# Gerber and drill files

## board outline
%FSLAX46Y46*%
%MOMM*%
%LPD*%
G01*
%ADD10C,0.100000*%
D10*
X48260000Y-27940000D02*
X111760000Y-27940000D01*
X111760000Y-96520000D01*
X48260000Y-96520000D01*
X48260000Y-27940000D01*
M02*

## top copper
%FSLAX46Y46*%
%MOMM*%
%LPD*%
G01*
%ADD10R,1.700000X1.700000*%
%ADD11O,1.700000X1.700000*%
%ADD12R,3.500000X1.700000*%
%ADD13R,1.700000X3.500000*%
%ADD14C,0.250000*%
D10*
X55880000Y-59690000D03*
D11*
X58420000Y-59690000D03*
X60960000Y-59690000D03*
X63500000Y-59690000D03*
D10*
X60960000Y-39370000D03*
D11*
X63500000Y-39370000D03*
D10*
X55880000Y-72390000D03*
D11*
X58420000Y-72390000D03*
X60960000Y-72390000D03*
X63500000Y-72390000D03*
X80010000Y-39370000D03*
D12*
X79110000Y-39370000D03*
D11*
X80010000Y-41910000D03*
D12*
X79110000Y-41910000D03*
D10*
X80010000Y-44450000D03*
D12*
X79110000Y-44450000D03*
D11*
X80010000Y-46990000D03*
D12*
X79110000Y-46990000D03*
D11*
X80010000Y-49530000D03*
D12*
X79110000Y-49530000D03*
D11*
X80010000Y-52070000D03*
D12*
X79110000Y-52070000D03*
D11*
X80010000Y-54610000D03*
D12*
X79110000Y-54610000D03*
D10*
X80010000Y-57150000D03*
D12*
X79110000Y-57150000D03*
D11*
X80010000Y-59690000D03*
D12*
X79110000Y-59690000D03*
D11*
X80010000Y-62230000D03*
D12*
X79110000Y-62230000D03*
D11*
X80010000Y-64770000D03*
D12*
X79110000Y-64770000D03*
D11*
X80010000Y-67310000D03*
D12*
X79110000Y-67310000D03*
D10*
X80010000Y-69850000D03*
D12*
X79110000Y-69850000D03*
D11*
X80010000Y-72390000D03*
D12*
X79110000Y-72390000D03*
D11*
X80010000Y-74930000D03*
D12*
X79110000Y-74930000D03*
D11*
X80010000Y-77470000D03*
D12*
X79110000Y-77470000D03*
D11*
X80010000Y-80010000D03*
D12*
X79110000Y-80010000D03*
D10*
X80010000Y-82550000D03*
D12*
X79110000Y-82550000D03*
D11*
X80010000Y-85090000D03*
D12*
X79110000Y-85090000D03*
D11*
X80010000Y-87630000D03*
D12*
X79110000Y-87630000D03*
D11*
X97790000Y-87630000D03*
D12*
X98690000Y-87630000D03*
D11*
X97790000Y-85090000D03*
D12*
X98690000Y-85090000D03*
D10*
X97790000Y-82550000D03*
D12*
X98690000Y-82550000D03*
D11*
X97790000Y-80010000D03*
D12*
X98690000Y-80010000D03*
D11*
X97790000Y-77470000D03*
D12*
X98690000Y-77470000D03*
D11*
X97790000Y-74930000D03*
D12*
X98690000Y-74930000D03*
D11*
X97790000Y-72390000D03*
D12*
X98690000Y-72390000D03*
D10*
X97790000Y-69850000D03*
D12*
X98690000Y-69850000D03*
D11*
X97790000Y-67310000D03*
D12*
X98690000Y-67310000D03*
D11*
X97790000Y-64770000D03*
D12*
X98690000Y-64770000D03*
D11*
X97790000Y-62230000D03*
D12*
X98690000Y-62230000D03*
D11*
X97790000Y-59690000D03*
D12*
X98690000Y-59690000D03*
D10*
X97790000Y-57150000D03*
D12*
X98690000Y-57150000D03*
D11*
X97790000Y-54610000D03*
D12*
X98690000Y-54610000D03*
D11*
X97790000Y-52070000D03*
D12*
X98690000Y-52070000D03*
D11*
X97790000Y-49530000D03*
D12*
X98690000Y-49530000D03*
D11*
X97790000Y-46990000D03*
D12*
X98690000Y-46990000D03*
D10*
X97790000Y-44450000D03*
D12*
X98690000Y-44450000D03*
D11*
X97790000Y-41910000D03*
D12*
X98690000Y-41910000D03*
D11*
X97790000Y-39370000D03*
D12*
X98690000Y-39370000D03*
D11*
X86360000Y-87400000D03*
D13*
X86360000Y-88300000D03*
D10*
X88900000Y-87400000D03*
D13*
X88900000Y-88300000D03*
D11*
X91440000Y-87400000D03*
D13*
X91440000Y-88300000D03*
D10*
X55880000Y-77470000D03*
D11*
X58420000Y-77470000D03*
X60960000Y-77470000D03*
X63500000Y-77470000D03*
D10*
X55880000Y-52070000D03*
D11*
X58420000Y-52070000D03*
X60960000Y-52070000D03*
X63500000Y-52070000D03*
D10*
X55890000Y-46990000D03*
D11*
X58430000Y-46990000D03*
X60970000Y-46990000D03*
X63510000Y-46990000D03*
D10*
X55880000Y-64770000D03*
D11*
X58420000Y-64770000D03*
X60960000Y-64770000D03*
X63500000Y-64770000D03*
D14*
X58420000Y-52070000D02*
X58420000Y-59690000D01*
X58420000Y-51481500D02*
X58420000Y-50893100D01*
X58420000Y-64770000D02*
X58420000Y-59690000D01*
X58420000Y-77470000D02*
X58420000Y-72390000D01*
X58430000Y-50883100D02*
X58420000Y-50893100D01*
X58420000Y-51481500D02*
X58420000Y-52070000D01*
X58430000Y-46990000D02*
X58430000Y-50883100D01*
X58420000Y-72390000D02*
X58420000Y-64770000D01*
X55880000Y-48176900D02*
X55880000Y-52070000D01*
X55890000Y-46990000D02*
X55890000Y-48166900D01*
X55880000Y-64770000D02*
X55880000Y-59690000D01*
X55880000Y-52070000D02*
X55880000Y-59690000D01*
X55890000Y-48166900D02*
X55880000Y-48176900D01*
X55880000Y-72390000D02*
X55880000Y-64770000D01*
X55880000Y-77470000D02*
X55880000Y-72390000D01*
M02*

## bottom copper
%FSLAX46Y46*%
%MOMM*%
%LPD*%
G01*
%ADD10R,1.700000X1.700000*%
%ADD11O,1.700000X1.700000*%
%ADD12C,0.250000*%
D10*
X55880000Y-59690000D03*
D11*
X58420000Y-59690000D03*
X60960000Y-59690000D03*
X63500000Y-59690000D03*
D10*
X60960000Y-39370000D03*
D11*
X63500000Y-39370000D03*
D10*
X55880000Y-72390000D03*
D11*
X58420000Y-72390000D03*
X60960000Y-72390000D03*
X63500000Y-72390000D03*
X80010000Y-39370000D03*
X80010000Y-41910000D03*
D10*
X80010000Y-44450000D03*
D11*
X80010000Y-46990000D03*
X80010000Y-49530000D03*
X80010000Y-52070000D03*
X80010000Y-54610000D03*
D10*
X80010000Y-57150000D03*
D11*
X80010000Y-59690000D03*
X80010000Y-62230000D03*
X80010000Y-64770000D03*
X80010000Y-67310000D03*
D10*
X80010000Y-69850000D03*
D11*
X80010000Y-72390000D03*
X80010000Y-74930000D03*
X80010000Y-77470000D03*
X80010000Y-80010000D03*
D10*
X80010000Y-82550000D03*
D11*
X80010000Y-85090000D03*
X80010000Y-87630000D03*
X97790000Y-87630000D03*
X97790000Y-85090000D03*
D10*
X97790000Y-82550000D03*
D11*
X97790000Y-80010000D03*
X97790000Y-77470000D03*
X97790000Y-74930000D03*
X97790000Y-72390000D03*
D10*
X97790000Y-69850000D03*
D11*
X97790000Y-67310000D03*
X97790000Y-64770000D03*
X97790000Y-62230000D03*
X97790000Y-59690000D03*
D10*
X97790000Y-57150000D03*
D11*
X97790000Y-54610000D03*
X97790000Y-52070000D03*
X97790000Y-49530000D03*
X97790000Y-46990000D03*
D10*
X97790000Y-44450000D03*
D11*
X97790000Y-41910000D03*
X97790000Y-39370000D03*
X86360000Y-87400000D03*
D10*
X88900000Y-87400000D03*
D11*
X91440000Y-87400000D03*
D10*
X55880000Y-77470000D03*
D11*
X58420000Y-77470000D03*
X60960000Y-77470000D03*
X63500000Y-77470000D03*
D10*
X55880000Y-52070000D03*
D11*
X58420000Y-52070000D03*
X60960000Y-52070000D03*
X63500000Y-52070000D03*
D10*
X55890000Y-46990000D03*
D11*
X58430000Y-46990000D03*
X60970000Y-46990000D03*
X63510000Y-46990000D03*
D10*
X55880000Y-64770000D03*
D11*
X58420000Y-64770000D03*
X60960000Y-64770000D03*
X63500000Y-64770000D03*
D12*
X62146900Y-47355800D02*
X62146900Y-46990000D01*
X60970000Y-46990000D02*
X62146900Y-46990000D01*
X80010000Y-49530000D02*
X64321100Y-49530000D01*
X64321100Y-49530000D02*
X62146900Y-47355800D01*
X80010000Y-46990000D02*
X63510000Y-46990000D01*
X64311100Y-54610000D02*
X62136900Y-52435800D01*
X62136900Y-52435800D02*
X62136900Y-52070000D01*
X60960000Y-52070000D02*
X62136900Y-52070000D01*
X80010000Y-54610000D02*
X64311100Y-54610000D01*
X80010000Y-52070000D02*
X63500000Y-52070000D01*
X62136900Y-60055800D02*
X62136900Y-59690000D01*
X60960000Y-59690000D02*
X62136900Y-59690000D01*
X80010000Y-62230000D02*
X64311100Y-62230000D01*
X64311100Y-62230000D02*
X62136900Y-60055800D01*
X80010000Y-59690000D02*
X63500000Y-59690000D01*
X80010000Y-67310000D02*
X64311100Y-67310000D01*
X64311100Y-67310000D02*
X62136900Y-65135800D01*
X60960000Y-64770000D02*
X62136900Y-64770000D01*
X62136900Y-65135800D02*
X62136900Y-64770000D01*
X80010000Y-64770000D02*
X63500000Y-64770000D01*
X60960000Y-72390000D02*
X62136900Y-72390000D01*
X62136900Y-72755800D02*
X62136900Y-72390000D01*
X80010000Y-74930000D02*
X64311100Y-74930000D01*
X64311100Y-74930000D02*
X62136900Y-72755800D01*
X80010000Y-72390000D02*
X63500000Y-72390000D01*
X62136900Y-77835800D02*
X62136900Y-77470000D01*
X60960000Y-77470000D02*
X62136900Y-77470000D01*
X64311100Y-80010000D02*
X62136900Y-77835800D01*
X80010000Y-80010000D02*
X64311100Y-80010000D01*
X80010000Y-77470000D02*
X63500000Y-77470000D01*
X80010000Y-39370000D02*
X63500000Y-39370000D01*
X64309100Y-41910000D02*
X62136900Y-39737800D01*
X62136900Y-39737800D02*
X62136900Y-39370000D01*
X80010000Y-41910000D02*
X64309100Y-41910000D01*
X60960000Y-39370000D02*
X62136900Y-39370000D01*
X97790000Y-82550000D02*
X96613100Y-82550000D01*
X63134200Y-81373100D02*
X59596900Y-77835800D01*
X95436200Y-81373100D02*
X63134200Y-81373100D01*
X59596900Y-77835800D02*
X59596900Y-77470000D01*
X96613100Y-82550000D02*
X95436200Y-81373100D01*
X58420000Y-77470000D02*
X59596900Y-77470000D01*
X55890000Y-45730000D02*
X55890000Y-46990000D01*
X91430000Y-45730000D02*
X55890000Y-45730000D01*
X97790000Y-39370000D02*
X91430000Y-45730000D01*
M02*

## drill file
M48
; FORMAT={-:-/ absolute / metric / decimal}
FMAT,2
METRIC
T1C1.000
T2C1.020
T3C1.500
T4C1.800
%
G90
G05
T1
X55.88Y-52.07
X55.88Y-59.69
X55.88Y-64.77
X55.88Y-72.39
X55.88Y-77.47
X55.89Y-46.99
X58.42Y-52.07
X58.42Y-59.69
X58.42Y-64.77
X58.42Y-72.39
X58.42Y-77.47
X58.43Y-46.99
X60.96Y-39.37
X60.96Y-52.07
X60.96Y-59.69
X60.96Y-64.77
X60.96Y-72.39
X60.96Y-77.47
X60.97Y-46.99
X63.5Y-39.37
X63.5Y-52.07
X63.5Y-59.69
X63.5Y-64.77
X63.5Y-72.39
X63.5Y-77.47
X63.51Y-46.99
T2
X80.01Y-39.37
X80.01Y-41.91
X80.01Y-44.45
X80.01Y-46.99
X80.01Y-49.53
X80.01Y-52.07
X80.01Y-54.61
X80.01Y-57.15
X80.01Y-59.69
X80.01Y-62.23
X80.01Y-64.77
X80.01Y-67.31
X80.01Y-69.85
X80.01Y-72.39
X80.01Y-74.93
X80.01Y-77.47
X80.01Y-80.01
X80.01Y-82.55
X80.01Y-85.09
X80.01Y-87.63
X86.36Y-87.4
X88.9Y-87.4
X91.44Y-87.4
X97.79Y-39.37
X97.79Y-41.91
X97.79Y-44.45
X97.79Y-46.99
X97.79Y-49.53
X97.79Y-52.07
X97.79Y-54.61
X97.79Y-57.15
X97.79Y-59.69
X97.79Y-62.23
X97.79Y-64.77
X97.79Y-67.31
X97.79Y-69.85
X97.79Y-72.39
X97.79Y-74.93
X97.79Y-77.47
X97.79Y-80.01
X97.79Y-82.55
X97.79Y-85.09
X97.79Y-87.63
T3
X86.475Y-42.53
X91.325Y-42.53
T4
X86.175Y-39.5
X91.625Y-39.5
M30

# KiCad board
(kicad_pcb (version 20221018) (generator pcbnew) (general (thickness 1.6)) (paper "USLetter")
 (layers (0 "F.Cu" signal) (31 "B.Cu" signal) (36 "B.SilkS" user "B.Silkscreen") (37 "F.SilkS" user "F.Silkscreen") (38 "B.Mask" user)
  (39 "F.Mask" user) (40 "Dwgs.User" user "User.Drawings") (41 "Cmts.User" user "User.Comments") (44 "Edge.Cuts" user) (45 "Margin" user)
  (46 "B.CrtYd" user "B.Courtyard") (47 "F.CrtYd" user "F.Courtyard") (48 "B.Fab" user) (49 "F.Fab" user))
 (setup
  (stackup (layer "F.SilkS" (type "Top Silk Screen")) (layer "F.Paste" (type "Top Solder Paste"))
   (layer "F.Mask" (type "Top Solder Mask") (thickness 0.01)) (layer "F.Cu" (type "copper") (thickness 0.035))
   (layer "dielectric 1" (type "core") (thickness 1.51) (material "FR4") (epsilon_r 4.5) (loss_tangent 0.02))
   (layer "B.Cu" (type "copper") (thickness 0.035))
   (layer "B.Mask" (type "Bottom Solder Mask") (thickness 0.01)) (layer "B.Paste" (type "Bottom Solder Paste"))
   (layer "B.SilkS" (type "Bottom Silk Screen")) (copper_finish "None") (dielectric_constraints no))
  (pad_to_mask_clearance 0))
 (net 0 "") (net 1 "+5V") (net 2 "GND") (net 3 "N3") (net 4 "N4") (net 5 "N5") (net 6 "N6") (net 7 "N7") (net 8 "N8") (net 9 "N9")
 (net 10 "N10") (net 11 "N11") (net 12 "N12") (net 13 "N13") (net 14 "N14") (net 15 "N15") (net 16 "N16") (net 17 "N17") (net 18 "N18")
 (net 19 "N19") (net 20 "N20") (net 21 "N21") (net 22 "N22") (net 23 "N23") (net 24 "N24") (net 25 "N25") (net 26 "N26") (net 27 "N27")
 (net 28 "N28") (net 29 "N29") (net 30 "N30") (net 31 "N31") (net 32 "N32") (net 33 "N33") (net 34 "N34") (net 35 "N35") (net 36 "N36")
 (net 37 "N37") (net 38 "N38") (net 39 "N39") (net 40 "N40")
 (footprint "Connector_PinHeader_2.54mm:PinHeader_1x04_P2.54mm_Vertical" (layer "F.Cu") (at 55.88 59.69 90)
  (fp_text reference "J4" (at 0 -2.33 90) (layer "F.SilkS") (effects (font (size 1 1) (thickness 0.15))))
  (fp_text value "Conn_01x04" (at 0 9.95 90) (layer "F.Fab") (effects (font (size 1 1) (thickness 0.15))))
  (pad "1" thru_hole rect (at 0 0 90) (size 1.7 1.7) (drill 1) (layers "*.Cu" "*.Mask") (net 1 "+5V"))
  (pad "2" thru_hole oval (at 0 2.54 90) (size 1.7 1.7) (drill 1) (layers "*.Cu" "*.Mask") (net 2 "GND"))
  (pad "3" thru_hole oval (at 0 5.08 90) (size 1.7 1.7) (drill 1) (layers "*.Cu" "*.Mask") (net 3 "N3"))
  (pad "4" thru_hole oval (at 0 7.62 90) (size 1.7 1.7) (drill 1) (layers "*.Cu" "*.Mask") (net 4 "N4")))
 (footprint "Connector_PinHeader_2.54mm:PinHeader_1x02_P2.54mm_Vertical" (layer "F.Cu") (at 60.96 39.37 90)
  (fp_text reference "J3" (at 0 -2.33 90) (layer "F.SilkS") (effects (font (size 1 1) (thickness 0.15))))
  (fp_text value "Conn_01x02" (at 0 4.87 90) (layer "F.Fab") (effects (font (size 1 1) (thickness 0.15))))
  (pad "1" thru_hole rect (at 0 0 90) (size 1.7 1.7) (drill 1) (layers "*.Cu" "*.Mask") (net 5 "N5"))
  (pad "2" thru_hole oval (at 0 2.54 90) (size 1.7 1.7) (drill 1) (layers "*.Cu" "*.Mask") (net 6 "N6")))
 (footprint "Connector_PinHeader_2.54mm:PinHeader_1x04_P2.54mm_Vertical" (layer "F.Cu") (at 55.88 72.39 90)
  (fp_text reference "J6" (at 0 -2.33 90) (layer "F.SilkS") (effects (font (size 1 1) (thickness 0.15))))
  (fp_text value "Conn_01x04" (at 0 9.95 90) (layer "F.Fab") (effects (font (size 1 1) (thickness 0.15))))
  (pad "1" thru_hole rect (at 0 0 90) (size 1.7 1.7) (drill 1) (layers "*.Cu" "*.Mask") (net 1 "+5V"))
  (pad "2" thru_hole oval (at 0 2.54 90) (size 1.7 1.7) (drill 1) (layers "*.Cu" "*.Mask") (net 2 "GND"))
  (pad "3" thru_hole oval (at 0 5.08 90) (size 1.7 1.7) (drill 1) (layers "*.Cu" "*.Mask") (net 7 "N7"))
  (pad "4" thru_hole oval (at 0 7.62 90) (size 1.7 1.7) (drill 1) (layers "*.Cu" "*.Mask") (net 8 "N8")))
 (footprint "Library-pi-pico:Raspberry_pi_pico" (layer "F.Cu") (at 91.794 24.13)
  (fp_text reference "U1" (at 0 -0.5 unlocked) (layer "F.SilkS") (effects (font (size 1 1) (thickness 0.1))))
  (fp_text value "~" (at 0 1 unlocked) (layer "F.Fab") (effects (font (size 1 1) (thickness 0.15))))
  (pad "" np_thru_hole oval (at -5.619 15.37) (size 1.8 1.8) (drill 1.8) (layers "*.Cu" "*.Mask"))
  (pad "" np_thru_hole oval (at -5.319 18.4) (size 1.5 1.5) (drill 1.5) (layers "*.Cu" "*.Mask"))
  (pad "" np_thru_hole oval (at -0.469 18.4) (size 1.5 1.5) (drill 1.5) (layers "*.Cu" "*.Mask"))
  (pad "" np_thru_hole oval (at -0.169 15.37) (size 1.8 1.8) (drill 1.8) (layers "*.Cu" "*.Mask"))
  (pad "1" thru_hole oval (at -11.784 15.24) (size 1.7 1.7) (drill 1.02) (layers "*.Cu" "*.Mask") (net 6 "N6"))
  (pad "1" smd rect (at -11.784 15.24) (size 3.5 1.7) (drill (offset -0.9 0)) (layers "F.Cu" "F.Mask") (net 6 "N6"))
  (pad "2" thru_hole oval (at -11.784 17.78) (size 1.7 1.7) (drill 1.02) (layers "*.Cu" "*.Mask") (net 5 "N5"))
  (pad "2" smd rect (at -11.784 17.78) (size 3.5 1.7) (drill (offset -0.9 0)) (layers "F.Cu" "F.Mask") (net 5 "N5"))
  (pad "3" thru_hole rect (at -11.784 20.32) (size 1.7 1.7) (drill 1.02) (layers "*.Cu" "*.Mask") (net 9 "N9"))
  (pad "3" smd rect (at -11.784 20.32) (size 3.5 1.7) (drill (offset -0.9 0)) (layers "F.Cu" "F.Mask") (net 9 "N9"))
  (pad "4" thru_hole oval (at -11.784 22.86) (size 1.7 1.7) (drill 1.02) (layers "*.Cu" "*.Mask") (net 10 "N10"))
  (pad "4" smd rect (at -11.784 22.86) (size 3.5 1.7) (drill (offset -0.9 0)) (layers "F.Cu" "F.Mask") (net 10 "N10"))
  (pad "5" thru_hole oval (at -11.784 25.4) (size 1.7 1.7) (drill 1.02) (layers "*.Cu" "*.Mask") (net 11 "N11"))
  (pad "5" smd rect (at -11.784 25.4) (size 3.5 1.7) (drill (offset -0.9 0)) (layers "F.Cu" "F.Mask") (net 11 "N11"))
  (pad "6" thru_hole oval (at -11.784 27.94) (size 1.7 1.7) (drill 1.02) (layers "*.Cu" "*.Mask") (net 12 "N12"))
  (pad "6" smd rect (at -11.784 27.94) (size 3.5 1.7) (drill (offset -0.9 0)) (layers "F.Cu" "F.Mask") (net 12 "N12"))
  (pad "7" thru_hole oval (at -11.784 30.48) (size 1.7 1.7) (drill 1.02) (layers "*.Cu" "*.Mask") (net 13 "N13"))
  (pad "7" smd rect (at -11.784 30.48) (size 3.5 1.7) (drill (offset -0.9 0)) (layers "F.Cu" "F.Mask") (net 13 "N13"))
  (pad "8" thru_hole rect (at -11.784 33.02) (size 1.7 1.7) (drill 1.02) (layers "*.Cu" "*.Mask") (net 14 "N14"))
  (pad "8" smd rect (at -11.784 33.02) (size 3.5 1.7) (drill (offset -0.9 0)) (layers "F.Cu" "F.Mask") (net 14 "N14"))
  (pad "9" thru_hole oval (at -11.784 35.56) (size 1.7 1.7) (drill 1.02) (layers "*.Cu" "*.Mask") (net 4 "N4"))
  (pad "9" smd rect (at -11.784 35.56) (size 3.5 1.7) (drill (offset -0.9 0)) (layers "F.Cu" "F.Mask") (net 4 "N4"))
  (pad "10" thru_hole oval (at -11.784 38.1) (size 1.7 1.7) (drill 1.02) (layers "*.Cu" "*.Mask") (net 3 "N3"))
  (pad "10" smd rect (at -11.784 38.1) (size 3.5 1.7) (drill (offset -0.9 0)) (layers "F.Cu" "F.Mask") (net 3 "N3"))
  (pad "11" thru_hole oval (at -11.784 40.64) (size 1.7 1.7) (drill 1.02) (layers "*.Cu" "*.Mask") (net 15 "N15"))
  (pad "11" smd rect (at -11.784 40.64) (size 3.5 1.7) (drill (offset -0.9 0)) (layers "F.Cu" "F.Mask") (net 15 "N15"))
  (pad "12" thru_hole oval (at -11.784 43.18) (size 1.7 1.7) (drill 1.02) (layers "*.Cu" "*.Mask") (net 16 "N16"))
  (pad "12" smd rect (at -11.784 43.18) (size 3.5 1.7) (drill (offset -0.9 0)) (layers "F.Cu" "F.Mask") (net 16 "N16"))
  (pad "13" thru_hole rect (at -11.784 45.72) (size 1.7 1.7) (drill 1.02) (layers "*.Cu" "*.Mask") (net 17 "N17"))
  (pad "13" smd rect (at -11.784 45.72) (size 3.5 1.7) (drill (offset -0.9 0)) (layers "F.Cu" "F.Mask") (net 17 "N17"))
  (pad "14" thru_hole oval (at -11.784 48.26) (size 1.7 1.7) (drill 1.02) (layers "*.Cu" "*.Mask") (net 8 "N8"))
  (pad "14" smd rect (at -11.784 48.26) (size 3.5 1.7) (drill (offset -0.9 0)) (layers "F.Cu" "F.Mask") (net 8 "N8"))
  (pad "15" thru_hole oval (at -11.784 50.8) (size 1.7 1.7) (drill 1.02) (layers "*.Cu" "*.Mask") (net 7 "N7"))
  (pad "15" smd rect (at -11.784 50.8) (size 3.5 1.7) (drill (offset -0.9 0)) (layers "F.Cu" "F.Mask") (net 7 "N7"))
  (pad "16" thru_hole oval (at -11.784 53.34) (size 1.7 1.7) (drill 1.02) (layers "*.Cu" "*.Mask") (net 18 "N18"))
  (pad "16" smd rect (at -11.784 53.34) (size 3.5 1.7) (drill (offset -0.9 0)) (layers "F.Cu" "F.Mask") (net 18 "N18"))
  (pad "17" thru_hole oval (at -11.784 55.88) (size 1.7 1.7) (drill 1.02) (layers "*.Cu" "*.Mask") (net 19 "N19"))
  (pad "17" smd rect (at -11.784 55.88) (size 3.5 1.7) (drill (offset -0.9 0)) (layers "F.Cu" "F.Mask") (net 19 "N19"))
  (pad "18" thru_hole rect (at -11.784 58.42) (size 1.7 1.7) (drill 1.02) (layers "*.Cu" "*.Mask") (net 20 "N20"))
  (pad "18" smd rect (at -11.784 58.42) (size 3.5 1.7) (drill (offset -0.9 0)) (layers "F.Cu" "F.Mask") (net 20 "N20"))
  (pad "19" thru_hole oval (at -11.784 60.96) (size 1.7 1.7) (drill 1.02) (layers "*.Cu" "*.Mask") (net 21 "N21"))
  (pad "19" smd rect (at -11.784 60.96) (size 3.5 1.7) (drill (offset -0.9 0)) (layers "F.Cu" "F.Mask") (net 21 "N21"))
  (pad "20" thru_hole oval (at -11.784 63.5) (size 1.7 1.7) (drill 1.02) (layers "*.Cu" "*.Mask") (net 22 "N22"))
  (pad "20" smd rect (at -11.784 63.5) (size 3.5 1.7) (drill (offset -0.9 0)) (layers "F.Cu" "F.Mask") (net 22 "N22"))
  (pad "21" thru_hole oval (at 5.996 63.5) (size 1.7 1.7) (drill 1.02) (layers "*.Cu" "*.Mask") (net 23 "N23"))
  (pad "21" smd rect (at 5.996 63.5) (size 3.5 1.7) (drill (offset 0.9 0)) (layers "F.Cu" "F.Mask") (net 23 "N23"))
  (pad "22" thru_hole oval (at 5.996 60.96) (size 1.7 1.7) (drill 1.02) (layers "*.Cu" "*.Mask") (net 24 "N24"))
  (pad "22" smd rect (at 5.996 60.96) (size 3.5 1.7) (drill (offset 0.9 0)) (layers "F.Cu" "F.Mask") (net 24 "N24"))
  (pad "23" thru_hole rect (at 5.996 58.42) (size 1.7 1.7) (drill 1.02) (layers "*.Cu" "*.Mask") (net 2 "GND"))
  (pad "23" smd rect (at 5.996 58.42) (size 3.5 1.7) (drill (offset 0.9 0)) (layers "F.Cu" "F.Mask") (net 2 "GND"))
  (pad "24" thru_hole oval (at 5.996 55.88) (size 1.7 1.7) (drill 1.02) (layers "*.Cu" "*.Mask") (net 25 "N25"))
  (pad "24" smd rect (at 5.996 55.88) (size 3.5 1.7) (drill (offset 0.9 0)) (layers "F.Cu" "F.Mask") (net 25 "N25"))
  (pad "25" thru_hole oval (at 5.996 53.34) (size 1.7 1.7) (drill 1.02) (layers "*.Cu" "*.Mask") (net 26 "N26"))
  (pad "25" smd rect (at 5.996 53.34) (size 3.5 1.7) (drill (offset 0.9 0)) (layers "F.Cu" "F.Mask") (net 26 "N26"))
  (pad "26" thru_hole oval (at 5.996 50.8) (size 1.7 1.7) (drill 1.02) (layers "*.Cu" "*.Mask") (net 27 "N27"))
  (pad "26" smd rect (at 5.996 50.8) (size 3.5 1.7) (drill (offset 0.9 0)) (layers "F.Cu" "F.Mask") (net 27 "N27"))
  (pad "27" thru_hole oval (at 5.996 48.26) (size 1.7 1.7) (drill 1.02) (layers "*.Cu" "*.Mask") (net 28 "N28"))
  (pad "27" smd rect (at 5.996 48.26) (size 3.5 1.7) (drill (offset 0.9 0)) (layers "F.Cu" "F.Mask") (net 28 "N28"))
  (pad "28" thru_hole rect (at 5.996 45.72) (size 1.7 1.7) (drill 1.02) (layers "*.Cu" "*.Mask") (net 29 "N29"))
  (pad "28" smd rect (at 5.996 45.72) (size 3.5 1.7) (drill (offset 0.9 0)) (layers "F.Cu" "F.Mask") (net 29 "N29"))
  (pad "29" thru_hole oval (at 5.996 43.18) (size 1.7 1.7) (drill 1.02) (layers "*.Cu" "*.Mask") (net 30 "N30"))
  (pad "29" smd rect (at 5.996 43.18) (size 3.5 1.7) (drill (offset 0.9 0)) (layers "F.Cu" "F.Mask") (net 30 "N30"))
  (pad "30" thru_hole oval (at 5.996 40.64) (size 1.7 1.7) (drill 1.02) (layers "*.Cu" "*.Mask") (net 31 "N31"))
  (pad "30" smd rect (at 5.996 40.64) (size 3.5 1.7) (drill (offset 0.9 0)) (layers "F.Cu" "F.Mask") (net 31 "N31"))
  (pad "31" thru_hole oval (at 5.996 38.1) (size 1.7 1.7) (drill 1.02) (layers "*.Cu" "*.Mask") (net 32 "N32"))
  (pad "31" smd rect (at 5.996 38.1) (size 3.5 1.7) (drill (offset 0.9 0)) (layers "F.Cu" "F.Mask") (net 32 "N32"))
  (pad "32" thru_hole oval (at 5.996 35.56) (size 1.7 1.7) (drill 1.02) (layers "*.Cu" "*.Mask") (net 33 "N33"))
  (pad "32" smd rect (at 5.996 35.56) (size 3.5 1.7) (drill (offset 0.9 0)) (layers "F.Cu" "F.Mask") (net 33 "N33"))
  (pad "33" thru_hole rect (at 5.996 33.02) (size 1.7 1.7) (drill 1.02) (layers "*.Cu" "*.Mask") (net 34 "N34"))
  (pad "33" smd rect (at 5.996 33.02) (size 3.5 1.7) (drill (offset 0.9 0)) (layers "F.Cu" "F.Mask") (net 34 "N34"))
  (pad "34" thru_hole oval (at 5.996 30.48) (size 1.7 1.7) (drill 1.02) (layers "*.Cu" "*.Mask") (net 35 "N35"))
  (pad "34" smd rect (at 5.996 30.48) (size 3.5 1.7) (drill (offset 0.9 0)) (layers "F.Cu" "F.Mask") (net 35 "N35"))
  (pad "35" thru_hole oval (at 5.996 27.94) (size 1.7 1.7) (drill 1.02) (layers "*.Cu" "*.Mask") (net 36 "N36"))
  (pad "35" smd rect (at 5.996 27.94) (size 3.5 1.7) (drill (offset 0.9 0)) (layers "F.Cu" "F.Mask") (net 36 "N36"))
  (pad "36" thru_hole oval (at 5.996 25.4) (size 1.7 1.7) (drill 1.02) (layers "*.Cu" "*.Mask") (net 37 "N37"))
  (pad "36" smd rect (at 5.996 25.4) (size 3.5 1.7) (drill (offset 0.9 0)) (layers "F.Cu" "F.Mask") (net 37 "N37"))
  (pad "37" thru_hole oval (at 5.996 22.86) (size 1.7 1.7) (drill 1.02) (layers "*.Cu" "*.Mask") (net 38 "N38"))
  (pad "37" smd rect (at 5.996 22.86) (size 3.5 1.7) (drill (offset 0.9 0)) (layers "F.Cu" "F.Mask") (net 38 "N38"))
  (pad "38" thru_hole rect (at 5.996 20.32) (size 1.7 1.7) (drill 1.02) (layers "*.Cu" "*.Mask") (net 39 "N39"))
  (pad "38" smd rect (at 5.996 20.32) (size 3.5 1.7) (drill (offset 0.9 0)) (layers "F.Cu" "F.Mask") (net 39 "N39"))
  (pad "39" thru_hole oval (at 5.996 17.78) (size 1.7 1.7) (drill 1.02) (layers "*.Cu" "*.Mask") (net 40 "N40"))
  (pad "39" smd rect (at 5.996 17.78) (size 3.5 1.7) (drill (offset 0.9 0)) (layers "F.Cu" "F.Mask") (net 40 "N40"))
  (pad "40" thru_hole oval (at 5.996 15.24) (size 1.7 1.7) (drill 1.02) (layers "*.Cu" "*.Mask") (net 1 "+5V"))
  (pad "40" smd rect (at 5.996 15.24) (size 3.5 1.7) (drill (offset 0.9 0)) (layers "F.Cu" "F.Mask") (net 1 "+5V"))
  (pad "41" thru_hole oval (at -5.434 63.27) (size 1.7 1.7) (drill 1.02) (layers "*.Cu" "*.Mask"))
  (pad "41" smd rect (at -5.434 63.27 90) (size 3.5 1.7) (drill (offset -0.9 0)) (layers "F.Cu" "F.Mask"))
  (pad "42" thru_hole rect (at -2.894 63.27) (size 1.7 1.7) (drill 1.02) (layers "*.Cu" "*.Mask"))
  (pad "42" smd rect (at -2.894 63.27 90) (size 3.5 1.7) (drill (offset -0.9 0)) (layers "F.Cu" "F.Mask"))
  (pad "43" thru_hole oval (at -0.354 63.27) (size 1.7 1.7) (drill 1.02) (layers "*.Cu" "*.Mask"))
  (pad "43" smd rect (at -0.354 63.27 90) (size 3.5 1.7) (drill (offset -0.9 0)) (layers "F.Cu" "F.Mask")))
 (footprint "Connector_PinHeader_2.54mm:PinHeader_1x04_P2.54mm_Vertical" (layer "F.Cu") (at 55.88 77.47 90)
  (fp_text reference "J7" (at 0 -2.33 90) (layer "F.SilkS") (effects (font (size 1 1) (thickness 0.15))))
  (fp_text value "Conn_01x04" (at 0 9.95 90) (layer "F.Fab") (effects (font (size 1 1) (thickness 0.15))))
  (pad "1" thru_hole rect (at 0 0 90) (size 1.7 1.7) (drill 1) (layers "*.Cu" "*.Mask") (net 1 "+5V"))
  (pad "2" thru_hole oval (at 0 2.54 90) (size 1.7 1.7) (drill 1) (layers "*.Cu" "*.Mask") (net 2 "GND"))
  (pad "3" thru_hole oval (at 0 5.08 90) (size 1.7 1.7) (drill 1) (layers "*.Cu" "*.Mask") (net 19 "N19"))
  (pad "4" thru_hole oval (at 0 7.62 90) (size 1.7 1.7) (drill 1) (layers "*.Cu" "*.Mask") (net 18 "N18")))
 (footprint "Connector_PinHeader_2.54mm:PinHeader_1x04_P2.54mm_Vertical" (layer "F.Cu") (at 55.88 52.07 90)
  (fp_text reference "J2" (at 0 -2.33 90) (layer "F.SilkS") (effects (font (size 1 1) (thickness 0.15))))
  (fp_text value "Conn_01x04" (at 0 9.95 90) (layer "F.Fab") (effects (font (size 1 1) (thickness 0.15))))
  (pad "1" thru_hole rect (at 0 0 90) (size 1.7 1.7) (drill 1) (layers "*.Cu" "*.Mask") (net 1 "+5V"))
  (pad "2" thru_hole oval (at 0 2.54 90) (size 1.7 1.7) (drill 1) (layers "*.Cu" "*.Mask") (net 2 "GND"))
  (pad "3" thru_hole oval (at 0 5.08 90) (size 1.7 1.7) (drill 1) (layers "*.Cu" "*.Mask") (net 13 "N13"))
  (pad "4" thru_hole oval (at 0 7.62 90) (size 1.7 1.7) (drill 1) (layers "*.Cu" "*.Mask") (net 12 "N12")))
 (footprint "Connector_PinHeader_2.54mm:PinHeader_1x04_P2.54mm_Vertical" (layer "F.Cu") (at 55.89 46.99 90)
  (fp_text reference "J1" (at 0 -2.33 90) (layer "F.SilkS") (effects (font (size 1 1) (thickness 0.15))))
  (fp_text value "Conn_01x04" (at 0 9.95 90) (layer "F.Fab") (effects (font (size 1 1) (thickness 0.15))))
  (pad "1" thru_hole rect (at 0 0 90) (size 1.7 1.7) (drill 1) (layers "*.Cu" "*.Mask") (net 1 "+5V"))
  (pad "2" thru_hole oval (at 0 2.54 90) (size 1.7 1.7) (drill 1) (layers "*.Cu" "*.Mask") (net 2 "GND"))
  (pad "3" thru_hole oval (at 0 5.08 90) (size 1.7 1.7) (drill 1) (layers "*.Cu" "*.Mask") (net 11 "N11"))
  (pad "4" thru_hole oval (at 0 7.62 90) (size 1.7 1.7) (drill 1) (layers "*.Cu" "*.Mask") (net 10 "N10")))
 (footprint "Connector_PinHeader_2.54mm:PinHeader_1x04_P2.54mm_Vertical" (layer "F.Cu") (at 55.88 64.77 90)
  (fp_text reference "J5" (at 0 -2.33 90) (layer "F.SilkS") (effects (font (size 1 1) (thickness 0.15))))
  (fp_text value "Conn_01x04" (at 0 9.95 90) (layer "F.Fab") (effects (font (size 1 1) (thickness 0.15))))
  (pad "1" thru_hole rect (at 0 0 90) (size 1.7 1.7) (drill 1) (layers "*.Cu" "*.Mask") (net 1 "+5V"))
  (pad "2" thru_hole oval (at 0 2.54 90) (size 1.7 1.7) (drill 1) (layers "*.Cu" "*.Mask") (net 2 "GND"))
  (pad "3" thru_hole oval (at 0 5.08 90) (size 1.7 1.7) (drill 1) (layers "*.Cu" "*.Mask") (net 16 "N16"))
  (pad "4" thru_hole oval (at 0 7.62 90) (size 1.7 1.7) (drill 1) (layers "*.Cu" "*.Mask") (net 15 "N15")))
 (gr_rect (start 48.26 27.94) (end 111.76 96.52) (stroke (width 0.1) (type default)) (fill none) (layer "Edge.Cuts"))
 (segment (start 62.1469 47.3558) (end 62.1469 46.99) (width 0.25) (layer "B.Cu") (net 11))
 (segment (start 60.97 46.99) (end 62.1469 46.99) (width 0.25) (layer "B.Cu") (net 11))
 (segment (start 80.01 49.53) (end 64.3211 49.53) (width 0.25) (layer "B.Cu") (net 11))
 (segment (start 64.3211 49.53) (end 62.1469 47.3558) (width 0.25) (layer "B.Cu") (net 11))
 (segment (start 80.01 46.99) (end 63.51 46.99) (width 0.25) (layer "B.Cu") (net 10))
 (segment (start 64.3111 54.61) (end 62.1369 52.4358) (width 0.25) (layer "B.Cu") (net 13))
 (segment (start 62.1369 52.4358) (end 62.1369 52.07) (width 0.25) (layer "B.Cu") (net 13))
 (segment (start 60.96 52.07) (end 62.1369 52.07) (width 0.25) (layer "B.Cu") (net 13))
 (segment (start 80.01 54.61) (end 64.3111 54.61) (width 0.25) (layer "B.Cu") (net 13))
 (segment (start 80.01 52.07) (end 63.5 52.07) (width 0.25) (layer "B.Cu") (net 12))
 (segment (start 62.1369 60.0558) (end 62.1369 59.69) (width 0.25) (layer "B.Cu") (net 3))
 (segment (start 60.96 59.69) (end 62.1369 59.69) (width 0.25) (layer "B.Cu") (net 3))
 (segment (start 80.01 62.23) (end 64.3111 62.23) (width 0.25) (layer "B.Cu") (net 3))
 (segment (start 64.3111 62.23) (end 62.1369 60.0558) (width 0.25) (layer "B.Cu") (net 3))
 (segment (start 80.01 59.69) (end 63.5 59.69) (width 0.25) (layer "B.Cu") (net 4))
 (segment (start 80.01 67.31) (end 64.3111 67.31) (width 0.25) (layer "B.Cu") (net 16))
 (segment (start 64.3111 67.31) (end 62.1369 65.1358) (width 0.25) (layer "B.Cu") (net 16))
 (segment (start 60.96 64.77) (end 62.1369 64.77) (width 0.25) (layer "B.Cu") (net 16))
 (segment (start 62.1369 65.1358) (end 62.1369 64.77) (width 0.25) (layer "B.Cu") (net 16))
 (segment (start 80.01 64.77) (end 63.5 64.77) (width 0.25) (layer "B.Cu") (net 15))
 (segment (start 60.96 72.39) (end 62.1369 72.39) (width 0.25) (layer "B.Cu") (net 7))
 (segment (start 62.1369 72.7558) (end 62.1369 72.39) (width 0.25) (layer "B.Cu") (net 7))
 (segment (start 80.01 74.93) (end 64.3111 74.93) (width 0.25) (layer "B.Cu") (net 7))
 (segment (start 64.3111 74.93) (end 62.1369 72.7558) (width 0.25) (layer "B.Cu") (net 7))
 (segment (start 80.01 72.39) (end 63.5 72.39) (width 0.25) (layer "B.Cu") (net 8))
 (segment (start 62.1369 77.8358) (end 62.1369 77.47) (width 0.25) (layer "B.Cu") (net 19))
 (segment (start 60.96 77.47) (end 62.1369 77.47) (width 0.25) (layer "B.Cu") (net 19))
 (segment (start 64.3111 80.01) (end 62.1369 77.8358) (width 0.25) (layer "B.Cu") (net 19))
 (segment (start 80.01 80.01) (end 64.3111 80.01) (width 0.25) (layer "B.Cu") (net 19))
 (segment (start 80.01 77.47) (end 63.5 77.47) (width 0.25) (layer "B.Cu") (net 18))
 (segment (start 80.01 39.37) (end 63.5 39.37) (width 0.25) (layer "B.Cu") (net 6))
 (segment (start 64.3091 41.91) (end 62.1369 39.7378) (width 0.25) (layer "B.Cu") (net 5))
 (segment (start 62.1369 39.7378) (end 62.1369 39.37) (width 0.25) (layer "B.Cu") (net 5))
 (segment (start 80.01 41.91) (end 64.3091 41.91) (width 0.25) (layer "B.Cu") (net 5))
 (segment (start 60.96 39.37) (end 62.1369 39.37) (width 0.25) (layer "B.Cu") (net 5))
 (segment (start 58.42 52.07) (end 58.42 59.69) (width 0.25) (layer "F.Cu") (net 2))
 (segment (start 58.42 51.4815) (end 58.42 50.8931) (width 0.25) (layer "F.Cu") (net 2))
 (segment (start 58.42 64.77) (end 58.42 59.69) (width 0.25) (layer "F.Cu") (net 2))
 (segment (start 58.42 77.47) (end 58.42 72.39) (width 0.25) (layer "F.Cu") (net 2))
 (segment (start 58.43 50.8831) (end 58.42 50.8931) (width 0.25) (layer "F.Cu") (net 2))
 (segment (start 58.42 51.4815) (end 58.42 52.07) (width 0.25) (layer "F.Cu") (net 2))
 (segment (start 58.43 46.99) (end 58.43 50.8831) (width 0.25) (layer "F.Cu") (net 2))
 (segment (start 58.42 72.39) (end 58.42 64.77) (width 0.25) (layer "F.Cu") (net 2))
 (segment (start 97.79 82.55) (end 96.6131 82.55) (width 0.25) (layer "B.Cu") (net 2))
 (segment (start 63.1342 81.3731) (end 59.5969 77.8358) (width 0.25) (layer "B.Cu") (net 2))
 (segment (start 95.4362 81.3731) (end 63.1342 81.3731) (width 0.25) (layer "B.Cu") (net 2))
 (segment (start 59.5969 77.8358) (end 59.5969 77.47) (width 0.25) (layer "B.Cu") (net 2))
 (segment (start 96.6131 82.55) (end 95.4362 81.3731) (width 0.25) (layer "B.Cu") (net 2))
 (segment (start 58.42 77.47) (end 59.5969 77.47) (width 0.25) (layer "B.Cu") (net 2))
 (segment (start 55.88 48.1769) (end 55.88 52.07) (width 0.25) (layer "F.Cu") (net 1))
 (segment (start 55.89 46.99) (end 55.89 48.1669) (width 0.25) (layer "F.Cu") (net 1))
 (segment (start 55.88 64.77) (end 55.88 59.69) (width 0.25) (layer "F.Cu") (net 1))
 (segment (start 55.88 52.07) (end 55.88 59.69) (width 0.25) (layer "F.Cu") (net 1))
 (segment (start 55.89 48.1669) (end 55.88 48.1769) (width 0.25) (layer "F.Cu") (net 1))
 (segment (start 55.88 72.39) (end 55.88 64.77) (width 0.25) (layer "F.Cu") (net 1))
 (segment (start 55.88 77.47) (end 55.88 72.39) (width 0.25) (layer "F.Cu") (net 1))
 (segment (start 55.89 45.73) (end 55.89 46.99) (width 0.25) (layer "B.Cu") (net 1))
 (segment (start 91.43 45.73) (end 55.89 45.73) (width 0.25) (layer "B.Cu") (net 1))
 (segment (start 97.79 39.37) (end 91.43 45.73) (width 0.25) (layer "B.Cu") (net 1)))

